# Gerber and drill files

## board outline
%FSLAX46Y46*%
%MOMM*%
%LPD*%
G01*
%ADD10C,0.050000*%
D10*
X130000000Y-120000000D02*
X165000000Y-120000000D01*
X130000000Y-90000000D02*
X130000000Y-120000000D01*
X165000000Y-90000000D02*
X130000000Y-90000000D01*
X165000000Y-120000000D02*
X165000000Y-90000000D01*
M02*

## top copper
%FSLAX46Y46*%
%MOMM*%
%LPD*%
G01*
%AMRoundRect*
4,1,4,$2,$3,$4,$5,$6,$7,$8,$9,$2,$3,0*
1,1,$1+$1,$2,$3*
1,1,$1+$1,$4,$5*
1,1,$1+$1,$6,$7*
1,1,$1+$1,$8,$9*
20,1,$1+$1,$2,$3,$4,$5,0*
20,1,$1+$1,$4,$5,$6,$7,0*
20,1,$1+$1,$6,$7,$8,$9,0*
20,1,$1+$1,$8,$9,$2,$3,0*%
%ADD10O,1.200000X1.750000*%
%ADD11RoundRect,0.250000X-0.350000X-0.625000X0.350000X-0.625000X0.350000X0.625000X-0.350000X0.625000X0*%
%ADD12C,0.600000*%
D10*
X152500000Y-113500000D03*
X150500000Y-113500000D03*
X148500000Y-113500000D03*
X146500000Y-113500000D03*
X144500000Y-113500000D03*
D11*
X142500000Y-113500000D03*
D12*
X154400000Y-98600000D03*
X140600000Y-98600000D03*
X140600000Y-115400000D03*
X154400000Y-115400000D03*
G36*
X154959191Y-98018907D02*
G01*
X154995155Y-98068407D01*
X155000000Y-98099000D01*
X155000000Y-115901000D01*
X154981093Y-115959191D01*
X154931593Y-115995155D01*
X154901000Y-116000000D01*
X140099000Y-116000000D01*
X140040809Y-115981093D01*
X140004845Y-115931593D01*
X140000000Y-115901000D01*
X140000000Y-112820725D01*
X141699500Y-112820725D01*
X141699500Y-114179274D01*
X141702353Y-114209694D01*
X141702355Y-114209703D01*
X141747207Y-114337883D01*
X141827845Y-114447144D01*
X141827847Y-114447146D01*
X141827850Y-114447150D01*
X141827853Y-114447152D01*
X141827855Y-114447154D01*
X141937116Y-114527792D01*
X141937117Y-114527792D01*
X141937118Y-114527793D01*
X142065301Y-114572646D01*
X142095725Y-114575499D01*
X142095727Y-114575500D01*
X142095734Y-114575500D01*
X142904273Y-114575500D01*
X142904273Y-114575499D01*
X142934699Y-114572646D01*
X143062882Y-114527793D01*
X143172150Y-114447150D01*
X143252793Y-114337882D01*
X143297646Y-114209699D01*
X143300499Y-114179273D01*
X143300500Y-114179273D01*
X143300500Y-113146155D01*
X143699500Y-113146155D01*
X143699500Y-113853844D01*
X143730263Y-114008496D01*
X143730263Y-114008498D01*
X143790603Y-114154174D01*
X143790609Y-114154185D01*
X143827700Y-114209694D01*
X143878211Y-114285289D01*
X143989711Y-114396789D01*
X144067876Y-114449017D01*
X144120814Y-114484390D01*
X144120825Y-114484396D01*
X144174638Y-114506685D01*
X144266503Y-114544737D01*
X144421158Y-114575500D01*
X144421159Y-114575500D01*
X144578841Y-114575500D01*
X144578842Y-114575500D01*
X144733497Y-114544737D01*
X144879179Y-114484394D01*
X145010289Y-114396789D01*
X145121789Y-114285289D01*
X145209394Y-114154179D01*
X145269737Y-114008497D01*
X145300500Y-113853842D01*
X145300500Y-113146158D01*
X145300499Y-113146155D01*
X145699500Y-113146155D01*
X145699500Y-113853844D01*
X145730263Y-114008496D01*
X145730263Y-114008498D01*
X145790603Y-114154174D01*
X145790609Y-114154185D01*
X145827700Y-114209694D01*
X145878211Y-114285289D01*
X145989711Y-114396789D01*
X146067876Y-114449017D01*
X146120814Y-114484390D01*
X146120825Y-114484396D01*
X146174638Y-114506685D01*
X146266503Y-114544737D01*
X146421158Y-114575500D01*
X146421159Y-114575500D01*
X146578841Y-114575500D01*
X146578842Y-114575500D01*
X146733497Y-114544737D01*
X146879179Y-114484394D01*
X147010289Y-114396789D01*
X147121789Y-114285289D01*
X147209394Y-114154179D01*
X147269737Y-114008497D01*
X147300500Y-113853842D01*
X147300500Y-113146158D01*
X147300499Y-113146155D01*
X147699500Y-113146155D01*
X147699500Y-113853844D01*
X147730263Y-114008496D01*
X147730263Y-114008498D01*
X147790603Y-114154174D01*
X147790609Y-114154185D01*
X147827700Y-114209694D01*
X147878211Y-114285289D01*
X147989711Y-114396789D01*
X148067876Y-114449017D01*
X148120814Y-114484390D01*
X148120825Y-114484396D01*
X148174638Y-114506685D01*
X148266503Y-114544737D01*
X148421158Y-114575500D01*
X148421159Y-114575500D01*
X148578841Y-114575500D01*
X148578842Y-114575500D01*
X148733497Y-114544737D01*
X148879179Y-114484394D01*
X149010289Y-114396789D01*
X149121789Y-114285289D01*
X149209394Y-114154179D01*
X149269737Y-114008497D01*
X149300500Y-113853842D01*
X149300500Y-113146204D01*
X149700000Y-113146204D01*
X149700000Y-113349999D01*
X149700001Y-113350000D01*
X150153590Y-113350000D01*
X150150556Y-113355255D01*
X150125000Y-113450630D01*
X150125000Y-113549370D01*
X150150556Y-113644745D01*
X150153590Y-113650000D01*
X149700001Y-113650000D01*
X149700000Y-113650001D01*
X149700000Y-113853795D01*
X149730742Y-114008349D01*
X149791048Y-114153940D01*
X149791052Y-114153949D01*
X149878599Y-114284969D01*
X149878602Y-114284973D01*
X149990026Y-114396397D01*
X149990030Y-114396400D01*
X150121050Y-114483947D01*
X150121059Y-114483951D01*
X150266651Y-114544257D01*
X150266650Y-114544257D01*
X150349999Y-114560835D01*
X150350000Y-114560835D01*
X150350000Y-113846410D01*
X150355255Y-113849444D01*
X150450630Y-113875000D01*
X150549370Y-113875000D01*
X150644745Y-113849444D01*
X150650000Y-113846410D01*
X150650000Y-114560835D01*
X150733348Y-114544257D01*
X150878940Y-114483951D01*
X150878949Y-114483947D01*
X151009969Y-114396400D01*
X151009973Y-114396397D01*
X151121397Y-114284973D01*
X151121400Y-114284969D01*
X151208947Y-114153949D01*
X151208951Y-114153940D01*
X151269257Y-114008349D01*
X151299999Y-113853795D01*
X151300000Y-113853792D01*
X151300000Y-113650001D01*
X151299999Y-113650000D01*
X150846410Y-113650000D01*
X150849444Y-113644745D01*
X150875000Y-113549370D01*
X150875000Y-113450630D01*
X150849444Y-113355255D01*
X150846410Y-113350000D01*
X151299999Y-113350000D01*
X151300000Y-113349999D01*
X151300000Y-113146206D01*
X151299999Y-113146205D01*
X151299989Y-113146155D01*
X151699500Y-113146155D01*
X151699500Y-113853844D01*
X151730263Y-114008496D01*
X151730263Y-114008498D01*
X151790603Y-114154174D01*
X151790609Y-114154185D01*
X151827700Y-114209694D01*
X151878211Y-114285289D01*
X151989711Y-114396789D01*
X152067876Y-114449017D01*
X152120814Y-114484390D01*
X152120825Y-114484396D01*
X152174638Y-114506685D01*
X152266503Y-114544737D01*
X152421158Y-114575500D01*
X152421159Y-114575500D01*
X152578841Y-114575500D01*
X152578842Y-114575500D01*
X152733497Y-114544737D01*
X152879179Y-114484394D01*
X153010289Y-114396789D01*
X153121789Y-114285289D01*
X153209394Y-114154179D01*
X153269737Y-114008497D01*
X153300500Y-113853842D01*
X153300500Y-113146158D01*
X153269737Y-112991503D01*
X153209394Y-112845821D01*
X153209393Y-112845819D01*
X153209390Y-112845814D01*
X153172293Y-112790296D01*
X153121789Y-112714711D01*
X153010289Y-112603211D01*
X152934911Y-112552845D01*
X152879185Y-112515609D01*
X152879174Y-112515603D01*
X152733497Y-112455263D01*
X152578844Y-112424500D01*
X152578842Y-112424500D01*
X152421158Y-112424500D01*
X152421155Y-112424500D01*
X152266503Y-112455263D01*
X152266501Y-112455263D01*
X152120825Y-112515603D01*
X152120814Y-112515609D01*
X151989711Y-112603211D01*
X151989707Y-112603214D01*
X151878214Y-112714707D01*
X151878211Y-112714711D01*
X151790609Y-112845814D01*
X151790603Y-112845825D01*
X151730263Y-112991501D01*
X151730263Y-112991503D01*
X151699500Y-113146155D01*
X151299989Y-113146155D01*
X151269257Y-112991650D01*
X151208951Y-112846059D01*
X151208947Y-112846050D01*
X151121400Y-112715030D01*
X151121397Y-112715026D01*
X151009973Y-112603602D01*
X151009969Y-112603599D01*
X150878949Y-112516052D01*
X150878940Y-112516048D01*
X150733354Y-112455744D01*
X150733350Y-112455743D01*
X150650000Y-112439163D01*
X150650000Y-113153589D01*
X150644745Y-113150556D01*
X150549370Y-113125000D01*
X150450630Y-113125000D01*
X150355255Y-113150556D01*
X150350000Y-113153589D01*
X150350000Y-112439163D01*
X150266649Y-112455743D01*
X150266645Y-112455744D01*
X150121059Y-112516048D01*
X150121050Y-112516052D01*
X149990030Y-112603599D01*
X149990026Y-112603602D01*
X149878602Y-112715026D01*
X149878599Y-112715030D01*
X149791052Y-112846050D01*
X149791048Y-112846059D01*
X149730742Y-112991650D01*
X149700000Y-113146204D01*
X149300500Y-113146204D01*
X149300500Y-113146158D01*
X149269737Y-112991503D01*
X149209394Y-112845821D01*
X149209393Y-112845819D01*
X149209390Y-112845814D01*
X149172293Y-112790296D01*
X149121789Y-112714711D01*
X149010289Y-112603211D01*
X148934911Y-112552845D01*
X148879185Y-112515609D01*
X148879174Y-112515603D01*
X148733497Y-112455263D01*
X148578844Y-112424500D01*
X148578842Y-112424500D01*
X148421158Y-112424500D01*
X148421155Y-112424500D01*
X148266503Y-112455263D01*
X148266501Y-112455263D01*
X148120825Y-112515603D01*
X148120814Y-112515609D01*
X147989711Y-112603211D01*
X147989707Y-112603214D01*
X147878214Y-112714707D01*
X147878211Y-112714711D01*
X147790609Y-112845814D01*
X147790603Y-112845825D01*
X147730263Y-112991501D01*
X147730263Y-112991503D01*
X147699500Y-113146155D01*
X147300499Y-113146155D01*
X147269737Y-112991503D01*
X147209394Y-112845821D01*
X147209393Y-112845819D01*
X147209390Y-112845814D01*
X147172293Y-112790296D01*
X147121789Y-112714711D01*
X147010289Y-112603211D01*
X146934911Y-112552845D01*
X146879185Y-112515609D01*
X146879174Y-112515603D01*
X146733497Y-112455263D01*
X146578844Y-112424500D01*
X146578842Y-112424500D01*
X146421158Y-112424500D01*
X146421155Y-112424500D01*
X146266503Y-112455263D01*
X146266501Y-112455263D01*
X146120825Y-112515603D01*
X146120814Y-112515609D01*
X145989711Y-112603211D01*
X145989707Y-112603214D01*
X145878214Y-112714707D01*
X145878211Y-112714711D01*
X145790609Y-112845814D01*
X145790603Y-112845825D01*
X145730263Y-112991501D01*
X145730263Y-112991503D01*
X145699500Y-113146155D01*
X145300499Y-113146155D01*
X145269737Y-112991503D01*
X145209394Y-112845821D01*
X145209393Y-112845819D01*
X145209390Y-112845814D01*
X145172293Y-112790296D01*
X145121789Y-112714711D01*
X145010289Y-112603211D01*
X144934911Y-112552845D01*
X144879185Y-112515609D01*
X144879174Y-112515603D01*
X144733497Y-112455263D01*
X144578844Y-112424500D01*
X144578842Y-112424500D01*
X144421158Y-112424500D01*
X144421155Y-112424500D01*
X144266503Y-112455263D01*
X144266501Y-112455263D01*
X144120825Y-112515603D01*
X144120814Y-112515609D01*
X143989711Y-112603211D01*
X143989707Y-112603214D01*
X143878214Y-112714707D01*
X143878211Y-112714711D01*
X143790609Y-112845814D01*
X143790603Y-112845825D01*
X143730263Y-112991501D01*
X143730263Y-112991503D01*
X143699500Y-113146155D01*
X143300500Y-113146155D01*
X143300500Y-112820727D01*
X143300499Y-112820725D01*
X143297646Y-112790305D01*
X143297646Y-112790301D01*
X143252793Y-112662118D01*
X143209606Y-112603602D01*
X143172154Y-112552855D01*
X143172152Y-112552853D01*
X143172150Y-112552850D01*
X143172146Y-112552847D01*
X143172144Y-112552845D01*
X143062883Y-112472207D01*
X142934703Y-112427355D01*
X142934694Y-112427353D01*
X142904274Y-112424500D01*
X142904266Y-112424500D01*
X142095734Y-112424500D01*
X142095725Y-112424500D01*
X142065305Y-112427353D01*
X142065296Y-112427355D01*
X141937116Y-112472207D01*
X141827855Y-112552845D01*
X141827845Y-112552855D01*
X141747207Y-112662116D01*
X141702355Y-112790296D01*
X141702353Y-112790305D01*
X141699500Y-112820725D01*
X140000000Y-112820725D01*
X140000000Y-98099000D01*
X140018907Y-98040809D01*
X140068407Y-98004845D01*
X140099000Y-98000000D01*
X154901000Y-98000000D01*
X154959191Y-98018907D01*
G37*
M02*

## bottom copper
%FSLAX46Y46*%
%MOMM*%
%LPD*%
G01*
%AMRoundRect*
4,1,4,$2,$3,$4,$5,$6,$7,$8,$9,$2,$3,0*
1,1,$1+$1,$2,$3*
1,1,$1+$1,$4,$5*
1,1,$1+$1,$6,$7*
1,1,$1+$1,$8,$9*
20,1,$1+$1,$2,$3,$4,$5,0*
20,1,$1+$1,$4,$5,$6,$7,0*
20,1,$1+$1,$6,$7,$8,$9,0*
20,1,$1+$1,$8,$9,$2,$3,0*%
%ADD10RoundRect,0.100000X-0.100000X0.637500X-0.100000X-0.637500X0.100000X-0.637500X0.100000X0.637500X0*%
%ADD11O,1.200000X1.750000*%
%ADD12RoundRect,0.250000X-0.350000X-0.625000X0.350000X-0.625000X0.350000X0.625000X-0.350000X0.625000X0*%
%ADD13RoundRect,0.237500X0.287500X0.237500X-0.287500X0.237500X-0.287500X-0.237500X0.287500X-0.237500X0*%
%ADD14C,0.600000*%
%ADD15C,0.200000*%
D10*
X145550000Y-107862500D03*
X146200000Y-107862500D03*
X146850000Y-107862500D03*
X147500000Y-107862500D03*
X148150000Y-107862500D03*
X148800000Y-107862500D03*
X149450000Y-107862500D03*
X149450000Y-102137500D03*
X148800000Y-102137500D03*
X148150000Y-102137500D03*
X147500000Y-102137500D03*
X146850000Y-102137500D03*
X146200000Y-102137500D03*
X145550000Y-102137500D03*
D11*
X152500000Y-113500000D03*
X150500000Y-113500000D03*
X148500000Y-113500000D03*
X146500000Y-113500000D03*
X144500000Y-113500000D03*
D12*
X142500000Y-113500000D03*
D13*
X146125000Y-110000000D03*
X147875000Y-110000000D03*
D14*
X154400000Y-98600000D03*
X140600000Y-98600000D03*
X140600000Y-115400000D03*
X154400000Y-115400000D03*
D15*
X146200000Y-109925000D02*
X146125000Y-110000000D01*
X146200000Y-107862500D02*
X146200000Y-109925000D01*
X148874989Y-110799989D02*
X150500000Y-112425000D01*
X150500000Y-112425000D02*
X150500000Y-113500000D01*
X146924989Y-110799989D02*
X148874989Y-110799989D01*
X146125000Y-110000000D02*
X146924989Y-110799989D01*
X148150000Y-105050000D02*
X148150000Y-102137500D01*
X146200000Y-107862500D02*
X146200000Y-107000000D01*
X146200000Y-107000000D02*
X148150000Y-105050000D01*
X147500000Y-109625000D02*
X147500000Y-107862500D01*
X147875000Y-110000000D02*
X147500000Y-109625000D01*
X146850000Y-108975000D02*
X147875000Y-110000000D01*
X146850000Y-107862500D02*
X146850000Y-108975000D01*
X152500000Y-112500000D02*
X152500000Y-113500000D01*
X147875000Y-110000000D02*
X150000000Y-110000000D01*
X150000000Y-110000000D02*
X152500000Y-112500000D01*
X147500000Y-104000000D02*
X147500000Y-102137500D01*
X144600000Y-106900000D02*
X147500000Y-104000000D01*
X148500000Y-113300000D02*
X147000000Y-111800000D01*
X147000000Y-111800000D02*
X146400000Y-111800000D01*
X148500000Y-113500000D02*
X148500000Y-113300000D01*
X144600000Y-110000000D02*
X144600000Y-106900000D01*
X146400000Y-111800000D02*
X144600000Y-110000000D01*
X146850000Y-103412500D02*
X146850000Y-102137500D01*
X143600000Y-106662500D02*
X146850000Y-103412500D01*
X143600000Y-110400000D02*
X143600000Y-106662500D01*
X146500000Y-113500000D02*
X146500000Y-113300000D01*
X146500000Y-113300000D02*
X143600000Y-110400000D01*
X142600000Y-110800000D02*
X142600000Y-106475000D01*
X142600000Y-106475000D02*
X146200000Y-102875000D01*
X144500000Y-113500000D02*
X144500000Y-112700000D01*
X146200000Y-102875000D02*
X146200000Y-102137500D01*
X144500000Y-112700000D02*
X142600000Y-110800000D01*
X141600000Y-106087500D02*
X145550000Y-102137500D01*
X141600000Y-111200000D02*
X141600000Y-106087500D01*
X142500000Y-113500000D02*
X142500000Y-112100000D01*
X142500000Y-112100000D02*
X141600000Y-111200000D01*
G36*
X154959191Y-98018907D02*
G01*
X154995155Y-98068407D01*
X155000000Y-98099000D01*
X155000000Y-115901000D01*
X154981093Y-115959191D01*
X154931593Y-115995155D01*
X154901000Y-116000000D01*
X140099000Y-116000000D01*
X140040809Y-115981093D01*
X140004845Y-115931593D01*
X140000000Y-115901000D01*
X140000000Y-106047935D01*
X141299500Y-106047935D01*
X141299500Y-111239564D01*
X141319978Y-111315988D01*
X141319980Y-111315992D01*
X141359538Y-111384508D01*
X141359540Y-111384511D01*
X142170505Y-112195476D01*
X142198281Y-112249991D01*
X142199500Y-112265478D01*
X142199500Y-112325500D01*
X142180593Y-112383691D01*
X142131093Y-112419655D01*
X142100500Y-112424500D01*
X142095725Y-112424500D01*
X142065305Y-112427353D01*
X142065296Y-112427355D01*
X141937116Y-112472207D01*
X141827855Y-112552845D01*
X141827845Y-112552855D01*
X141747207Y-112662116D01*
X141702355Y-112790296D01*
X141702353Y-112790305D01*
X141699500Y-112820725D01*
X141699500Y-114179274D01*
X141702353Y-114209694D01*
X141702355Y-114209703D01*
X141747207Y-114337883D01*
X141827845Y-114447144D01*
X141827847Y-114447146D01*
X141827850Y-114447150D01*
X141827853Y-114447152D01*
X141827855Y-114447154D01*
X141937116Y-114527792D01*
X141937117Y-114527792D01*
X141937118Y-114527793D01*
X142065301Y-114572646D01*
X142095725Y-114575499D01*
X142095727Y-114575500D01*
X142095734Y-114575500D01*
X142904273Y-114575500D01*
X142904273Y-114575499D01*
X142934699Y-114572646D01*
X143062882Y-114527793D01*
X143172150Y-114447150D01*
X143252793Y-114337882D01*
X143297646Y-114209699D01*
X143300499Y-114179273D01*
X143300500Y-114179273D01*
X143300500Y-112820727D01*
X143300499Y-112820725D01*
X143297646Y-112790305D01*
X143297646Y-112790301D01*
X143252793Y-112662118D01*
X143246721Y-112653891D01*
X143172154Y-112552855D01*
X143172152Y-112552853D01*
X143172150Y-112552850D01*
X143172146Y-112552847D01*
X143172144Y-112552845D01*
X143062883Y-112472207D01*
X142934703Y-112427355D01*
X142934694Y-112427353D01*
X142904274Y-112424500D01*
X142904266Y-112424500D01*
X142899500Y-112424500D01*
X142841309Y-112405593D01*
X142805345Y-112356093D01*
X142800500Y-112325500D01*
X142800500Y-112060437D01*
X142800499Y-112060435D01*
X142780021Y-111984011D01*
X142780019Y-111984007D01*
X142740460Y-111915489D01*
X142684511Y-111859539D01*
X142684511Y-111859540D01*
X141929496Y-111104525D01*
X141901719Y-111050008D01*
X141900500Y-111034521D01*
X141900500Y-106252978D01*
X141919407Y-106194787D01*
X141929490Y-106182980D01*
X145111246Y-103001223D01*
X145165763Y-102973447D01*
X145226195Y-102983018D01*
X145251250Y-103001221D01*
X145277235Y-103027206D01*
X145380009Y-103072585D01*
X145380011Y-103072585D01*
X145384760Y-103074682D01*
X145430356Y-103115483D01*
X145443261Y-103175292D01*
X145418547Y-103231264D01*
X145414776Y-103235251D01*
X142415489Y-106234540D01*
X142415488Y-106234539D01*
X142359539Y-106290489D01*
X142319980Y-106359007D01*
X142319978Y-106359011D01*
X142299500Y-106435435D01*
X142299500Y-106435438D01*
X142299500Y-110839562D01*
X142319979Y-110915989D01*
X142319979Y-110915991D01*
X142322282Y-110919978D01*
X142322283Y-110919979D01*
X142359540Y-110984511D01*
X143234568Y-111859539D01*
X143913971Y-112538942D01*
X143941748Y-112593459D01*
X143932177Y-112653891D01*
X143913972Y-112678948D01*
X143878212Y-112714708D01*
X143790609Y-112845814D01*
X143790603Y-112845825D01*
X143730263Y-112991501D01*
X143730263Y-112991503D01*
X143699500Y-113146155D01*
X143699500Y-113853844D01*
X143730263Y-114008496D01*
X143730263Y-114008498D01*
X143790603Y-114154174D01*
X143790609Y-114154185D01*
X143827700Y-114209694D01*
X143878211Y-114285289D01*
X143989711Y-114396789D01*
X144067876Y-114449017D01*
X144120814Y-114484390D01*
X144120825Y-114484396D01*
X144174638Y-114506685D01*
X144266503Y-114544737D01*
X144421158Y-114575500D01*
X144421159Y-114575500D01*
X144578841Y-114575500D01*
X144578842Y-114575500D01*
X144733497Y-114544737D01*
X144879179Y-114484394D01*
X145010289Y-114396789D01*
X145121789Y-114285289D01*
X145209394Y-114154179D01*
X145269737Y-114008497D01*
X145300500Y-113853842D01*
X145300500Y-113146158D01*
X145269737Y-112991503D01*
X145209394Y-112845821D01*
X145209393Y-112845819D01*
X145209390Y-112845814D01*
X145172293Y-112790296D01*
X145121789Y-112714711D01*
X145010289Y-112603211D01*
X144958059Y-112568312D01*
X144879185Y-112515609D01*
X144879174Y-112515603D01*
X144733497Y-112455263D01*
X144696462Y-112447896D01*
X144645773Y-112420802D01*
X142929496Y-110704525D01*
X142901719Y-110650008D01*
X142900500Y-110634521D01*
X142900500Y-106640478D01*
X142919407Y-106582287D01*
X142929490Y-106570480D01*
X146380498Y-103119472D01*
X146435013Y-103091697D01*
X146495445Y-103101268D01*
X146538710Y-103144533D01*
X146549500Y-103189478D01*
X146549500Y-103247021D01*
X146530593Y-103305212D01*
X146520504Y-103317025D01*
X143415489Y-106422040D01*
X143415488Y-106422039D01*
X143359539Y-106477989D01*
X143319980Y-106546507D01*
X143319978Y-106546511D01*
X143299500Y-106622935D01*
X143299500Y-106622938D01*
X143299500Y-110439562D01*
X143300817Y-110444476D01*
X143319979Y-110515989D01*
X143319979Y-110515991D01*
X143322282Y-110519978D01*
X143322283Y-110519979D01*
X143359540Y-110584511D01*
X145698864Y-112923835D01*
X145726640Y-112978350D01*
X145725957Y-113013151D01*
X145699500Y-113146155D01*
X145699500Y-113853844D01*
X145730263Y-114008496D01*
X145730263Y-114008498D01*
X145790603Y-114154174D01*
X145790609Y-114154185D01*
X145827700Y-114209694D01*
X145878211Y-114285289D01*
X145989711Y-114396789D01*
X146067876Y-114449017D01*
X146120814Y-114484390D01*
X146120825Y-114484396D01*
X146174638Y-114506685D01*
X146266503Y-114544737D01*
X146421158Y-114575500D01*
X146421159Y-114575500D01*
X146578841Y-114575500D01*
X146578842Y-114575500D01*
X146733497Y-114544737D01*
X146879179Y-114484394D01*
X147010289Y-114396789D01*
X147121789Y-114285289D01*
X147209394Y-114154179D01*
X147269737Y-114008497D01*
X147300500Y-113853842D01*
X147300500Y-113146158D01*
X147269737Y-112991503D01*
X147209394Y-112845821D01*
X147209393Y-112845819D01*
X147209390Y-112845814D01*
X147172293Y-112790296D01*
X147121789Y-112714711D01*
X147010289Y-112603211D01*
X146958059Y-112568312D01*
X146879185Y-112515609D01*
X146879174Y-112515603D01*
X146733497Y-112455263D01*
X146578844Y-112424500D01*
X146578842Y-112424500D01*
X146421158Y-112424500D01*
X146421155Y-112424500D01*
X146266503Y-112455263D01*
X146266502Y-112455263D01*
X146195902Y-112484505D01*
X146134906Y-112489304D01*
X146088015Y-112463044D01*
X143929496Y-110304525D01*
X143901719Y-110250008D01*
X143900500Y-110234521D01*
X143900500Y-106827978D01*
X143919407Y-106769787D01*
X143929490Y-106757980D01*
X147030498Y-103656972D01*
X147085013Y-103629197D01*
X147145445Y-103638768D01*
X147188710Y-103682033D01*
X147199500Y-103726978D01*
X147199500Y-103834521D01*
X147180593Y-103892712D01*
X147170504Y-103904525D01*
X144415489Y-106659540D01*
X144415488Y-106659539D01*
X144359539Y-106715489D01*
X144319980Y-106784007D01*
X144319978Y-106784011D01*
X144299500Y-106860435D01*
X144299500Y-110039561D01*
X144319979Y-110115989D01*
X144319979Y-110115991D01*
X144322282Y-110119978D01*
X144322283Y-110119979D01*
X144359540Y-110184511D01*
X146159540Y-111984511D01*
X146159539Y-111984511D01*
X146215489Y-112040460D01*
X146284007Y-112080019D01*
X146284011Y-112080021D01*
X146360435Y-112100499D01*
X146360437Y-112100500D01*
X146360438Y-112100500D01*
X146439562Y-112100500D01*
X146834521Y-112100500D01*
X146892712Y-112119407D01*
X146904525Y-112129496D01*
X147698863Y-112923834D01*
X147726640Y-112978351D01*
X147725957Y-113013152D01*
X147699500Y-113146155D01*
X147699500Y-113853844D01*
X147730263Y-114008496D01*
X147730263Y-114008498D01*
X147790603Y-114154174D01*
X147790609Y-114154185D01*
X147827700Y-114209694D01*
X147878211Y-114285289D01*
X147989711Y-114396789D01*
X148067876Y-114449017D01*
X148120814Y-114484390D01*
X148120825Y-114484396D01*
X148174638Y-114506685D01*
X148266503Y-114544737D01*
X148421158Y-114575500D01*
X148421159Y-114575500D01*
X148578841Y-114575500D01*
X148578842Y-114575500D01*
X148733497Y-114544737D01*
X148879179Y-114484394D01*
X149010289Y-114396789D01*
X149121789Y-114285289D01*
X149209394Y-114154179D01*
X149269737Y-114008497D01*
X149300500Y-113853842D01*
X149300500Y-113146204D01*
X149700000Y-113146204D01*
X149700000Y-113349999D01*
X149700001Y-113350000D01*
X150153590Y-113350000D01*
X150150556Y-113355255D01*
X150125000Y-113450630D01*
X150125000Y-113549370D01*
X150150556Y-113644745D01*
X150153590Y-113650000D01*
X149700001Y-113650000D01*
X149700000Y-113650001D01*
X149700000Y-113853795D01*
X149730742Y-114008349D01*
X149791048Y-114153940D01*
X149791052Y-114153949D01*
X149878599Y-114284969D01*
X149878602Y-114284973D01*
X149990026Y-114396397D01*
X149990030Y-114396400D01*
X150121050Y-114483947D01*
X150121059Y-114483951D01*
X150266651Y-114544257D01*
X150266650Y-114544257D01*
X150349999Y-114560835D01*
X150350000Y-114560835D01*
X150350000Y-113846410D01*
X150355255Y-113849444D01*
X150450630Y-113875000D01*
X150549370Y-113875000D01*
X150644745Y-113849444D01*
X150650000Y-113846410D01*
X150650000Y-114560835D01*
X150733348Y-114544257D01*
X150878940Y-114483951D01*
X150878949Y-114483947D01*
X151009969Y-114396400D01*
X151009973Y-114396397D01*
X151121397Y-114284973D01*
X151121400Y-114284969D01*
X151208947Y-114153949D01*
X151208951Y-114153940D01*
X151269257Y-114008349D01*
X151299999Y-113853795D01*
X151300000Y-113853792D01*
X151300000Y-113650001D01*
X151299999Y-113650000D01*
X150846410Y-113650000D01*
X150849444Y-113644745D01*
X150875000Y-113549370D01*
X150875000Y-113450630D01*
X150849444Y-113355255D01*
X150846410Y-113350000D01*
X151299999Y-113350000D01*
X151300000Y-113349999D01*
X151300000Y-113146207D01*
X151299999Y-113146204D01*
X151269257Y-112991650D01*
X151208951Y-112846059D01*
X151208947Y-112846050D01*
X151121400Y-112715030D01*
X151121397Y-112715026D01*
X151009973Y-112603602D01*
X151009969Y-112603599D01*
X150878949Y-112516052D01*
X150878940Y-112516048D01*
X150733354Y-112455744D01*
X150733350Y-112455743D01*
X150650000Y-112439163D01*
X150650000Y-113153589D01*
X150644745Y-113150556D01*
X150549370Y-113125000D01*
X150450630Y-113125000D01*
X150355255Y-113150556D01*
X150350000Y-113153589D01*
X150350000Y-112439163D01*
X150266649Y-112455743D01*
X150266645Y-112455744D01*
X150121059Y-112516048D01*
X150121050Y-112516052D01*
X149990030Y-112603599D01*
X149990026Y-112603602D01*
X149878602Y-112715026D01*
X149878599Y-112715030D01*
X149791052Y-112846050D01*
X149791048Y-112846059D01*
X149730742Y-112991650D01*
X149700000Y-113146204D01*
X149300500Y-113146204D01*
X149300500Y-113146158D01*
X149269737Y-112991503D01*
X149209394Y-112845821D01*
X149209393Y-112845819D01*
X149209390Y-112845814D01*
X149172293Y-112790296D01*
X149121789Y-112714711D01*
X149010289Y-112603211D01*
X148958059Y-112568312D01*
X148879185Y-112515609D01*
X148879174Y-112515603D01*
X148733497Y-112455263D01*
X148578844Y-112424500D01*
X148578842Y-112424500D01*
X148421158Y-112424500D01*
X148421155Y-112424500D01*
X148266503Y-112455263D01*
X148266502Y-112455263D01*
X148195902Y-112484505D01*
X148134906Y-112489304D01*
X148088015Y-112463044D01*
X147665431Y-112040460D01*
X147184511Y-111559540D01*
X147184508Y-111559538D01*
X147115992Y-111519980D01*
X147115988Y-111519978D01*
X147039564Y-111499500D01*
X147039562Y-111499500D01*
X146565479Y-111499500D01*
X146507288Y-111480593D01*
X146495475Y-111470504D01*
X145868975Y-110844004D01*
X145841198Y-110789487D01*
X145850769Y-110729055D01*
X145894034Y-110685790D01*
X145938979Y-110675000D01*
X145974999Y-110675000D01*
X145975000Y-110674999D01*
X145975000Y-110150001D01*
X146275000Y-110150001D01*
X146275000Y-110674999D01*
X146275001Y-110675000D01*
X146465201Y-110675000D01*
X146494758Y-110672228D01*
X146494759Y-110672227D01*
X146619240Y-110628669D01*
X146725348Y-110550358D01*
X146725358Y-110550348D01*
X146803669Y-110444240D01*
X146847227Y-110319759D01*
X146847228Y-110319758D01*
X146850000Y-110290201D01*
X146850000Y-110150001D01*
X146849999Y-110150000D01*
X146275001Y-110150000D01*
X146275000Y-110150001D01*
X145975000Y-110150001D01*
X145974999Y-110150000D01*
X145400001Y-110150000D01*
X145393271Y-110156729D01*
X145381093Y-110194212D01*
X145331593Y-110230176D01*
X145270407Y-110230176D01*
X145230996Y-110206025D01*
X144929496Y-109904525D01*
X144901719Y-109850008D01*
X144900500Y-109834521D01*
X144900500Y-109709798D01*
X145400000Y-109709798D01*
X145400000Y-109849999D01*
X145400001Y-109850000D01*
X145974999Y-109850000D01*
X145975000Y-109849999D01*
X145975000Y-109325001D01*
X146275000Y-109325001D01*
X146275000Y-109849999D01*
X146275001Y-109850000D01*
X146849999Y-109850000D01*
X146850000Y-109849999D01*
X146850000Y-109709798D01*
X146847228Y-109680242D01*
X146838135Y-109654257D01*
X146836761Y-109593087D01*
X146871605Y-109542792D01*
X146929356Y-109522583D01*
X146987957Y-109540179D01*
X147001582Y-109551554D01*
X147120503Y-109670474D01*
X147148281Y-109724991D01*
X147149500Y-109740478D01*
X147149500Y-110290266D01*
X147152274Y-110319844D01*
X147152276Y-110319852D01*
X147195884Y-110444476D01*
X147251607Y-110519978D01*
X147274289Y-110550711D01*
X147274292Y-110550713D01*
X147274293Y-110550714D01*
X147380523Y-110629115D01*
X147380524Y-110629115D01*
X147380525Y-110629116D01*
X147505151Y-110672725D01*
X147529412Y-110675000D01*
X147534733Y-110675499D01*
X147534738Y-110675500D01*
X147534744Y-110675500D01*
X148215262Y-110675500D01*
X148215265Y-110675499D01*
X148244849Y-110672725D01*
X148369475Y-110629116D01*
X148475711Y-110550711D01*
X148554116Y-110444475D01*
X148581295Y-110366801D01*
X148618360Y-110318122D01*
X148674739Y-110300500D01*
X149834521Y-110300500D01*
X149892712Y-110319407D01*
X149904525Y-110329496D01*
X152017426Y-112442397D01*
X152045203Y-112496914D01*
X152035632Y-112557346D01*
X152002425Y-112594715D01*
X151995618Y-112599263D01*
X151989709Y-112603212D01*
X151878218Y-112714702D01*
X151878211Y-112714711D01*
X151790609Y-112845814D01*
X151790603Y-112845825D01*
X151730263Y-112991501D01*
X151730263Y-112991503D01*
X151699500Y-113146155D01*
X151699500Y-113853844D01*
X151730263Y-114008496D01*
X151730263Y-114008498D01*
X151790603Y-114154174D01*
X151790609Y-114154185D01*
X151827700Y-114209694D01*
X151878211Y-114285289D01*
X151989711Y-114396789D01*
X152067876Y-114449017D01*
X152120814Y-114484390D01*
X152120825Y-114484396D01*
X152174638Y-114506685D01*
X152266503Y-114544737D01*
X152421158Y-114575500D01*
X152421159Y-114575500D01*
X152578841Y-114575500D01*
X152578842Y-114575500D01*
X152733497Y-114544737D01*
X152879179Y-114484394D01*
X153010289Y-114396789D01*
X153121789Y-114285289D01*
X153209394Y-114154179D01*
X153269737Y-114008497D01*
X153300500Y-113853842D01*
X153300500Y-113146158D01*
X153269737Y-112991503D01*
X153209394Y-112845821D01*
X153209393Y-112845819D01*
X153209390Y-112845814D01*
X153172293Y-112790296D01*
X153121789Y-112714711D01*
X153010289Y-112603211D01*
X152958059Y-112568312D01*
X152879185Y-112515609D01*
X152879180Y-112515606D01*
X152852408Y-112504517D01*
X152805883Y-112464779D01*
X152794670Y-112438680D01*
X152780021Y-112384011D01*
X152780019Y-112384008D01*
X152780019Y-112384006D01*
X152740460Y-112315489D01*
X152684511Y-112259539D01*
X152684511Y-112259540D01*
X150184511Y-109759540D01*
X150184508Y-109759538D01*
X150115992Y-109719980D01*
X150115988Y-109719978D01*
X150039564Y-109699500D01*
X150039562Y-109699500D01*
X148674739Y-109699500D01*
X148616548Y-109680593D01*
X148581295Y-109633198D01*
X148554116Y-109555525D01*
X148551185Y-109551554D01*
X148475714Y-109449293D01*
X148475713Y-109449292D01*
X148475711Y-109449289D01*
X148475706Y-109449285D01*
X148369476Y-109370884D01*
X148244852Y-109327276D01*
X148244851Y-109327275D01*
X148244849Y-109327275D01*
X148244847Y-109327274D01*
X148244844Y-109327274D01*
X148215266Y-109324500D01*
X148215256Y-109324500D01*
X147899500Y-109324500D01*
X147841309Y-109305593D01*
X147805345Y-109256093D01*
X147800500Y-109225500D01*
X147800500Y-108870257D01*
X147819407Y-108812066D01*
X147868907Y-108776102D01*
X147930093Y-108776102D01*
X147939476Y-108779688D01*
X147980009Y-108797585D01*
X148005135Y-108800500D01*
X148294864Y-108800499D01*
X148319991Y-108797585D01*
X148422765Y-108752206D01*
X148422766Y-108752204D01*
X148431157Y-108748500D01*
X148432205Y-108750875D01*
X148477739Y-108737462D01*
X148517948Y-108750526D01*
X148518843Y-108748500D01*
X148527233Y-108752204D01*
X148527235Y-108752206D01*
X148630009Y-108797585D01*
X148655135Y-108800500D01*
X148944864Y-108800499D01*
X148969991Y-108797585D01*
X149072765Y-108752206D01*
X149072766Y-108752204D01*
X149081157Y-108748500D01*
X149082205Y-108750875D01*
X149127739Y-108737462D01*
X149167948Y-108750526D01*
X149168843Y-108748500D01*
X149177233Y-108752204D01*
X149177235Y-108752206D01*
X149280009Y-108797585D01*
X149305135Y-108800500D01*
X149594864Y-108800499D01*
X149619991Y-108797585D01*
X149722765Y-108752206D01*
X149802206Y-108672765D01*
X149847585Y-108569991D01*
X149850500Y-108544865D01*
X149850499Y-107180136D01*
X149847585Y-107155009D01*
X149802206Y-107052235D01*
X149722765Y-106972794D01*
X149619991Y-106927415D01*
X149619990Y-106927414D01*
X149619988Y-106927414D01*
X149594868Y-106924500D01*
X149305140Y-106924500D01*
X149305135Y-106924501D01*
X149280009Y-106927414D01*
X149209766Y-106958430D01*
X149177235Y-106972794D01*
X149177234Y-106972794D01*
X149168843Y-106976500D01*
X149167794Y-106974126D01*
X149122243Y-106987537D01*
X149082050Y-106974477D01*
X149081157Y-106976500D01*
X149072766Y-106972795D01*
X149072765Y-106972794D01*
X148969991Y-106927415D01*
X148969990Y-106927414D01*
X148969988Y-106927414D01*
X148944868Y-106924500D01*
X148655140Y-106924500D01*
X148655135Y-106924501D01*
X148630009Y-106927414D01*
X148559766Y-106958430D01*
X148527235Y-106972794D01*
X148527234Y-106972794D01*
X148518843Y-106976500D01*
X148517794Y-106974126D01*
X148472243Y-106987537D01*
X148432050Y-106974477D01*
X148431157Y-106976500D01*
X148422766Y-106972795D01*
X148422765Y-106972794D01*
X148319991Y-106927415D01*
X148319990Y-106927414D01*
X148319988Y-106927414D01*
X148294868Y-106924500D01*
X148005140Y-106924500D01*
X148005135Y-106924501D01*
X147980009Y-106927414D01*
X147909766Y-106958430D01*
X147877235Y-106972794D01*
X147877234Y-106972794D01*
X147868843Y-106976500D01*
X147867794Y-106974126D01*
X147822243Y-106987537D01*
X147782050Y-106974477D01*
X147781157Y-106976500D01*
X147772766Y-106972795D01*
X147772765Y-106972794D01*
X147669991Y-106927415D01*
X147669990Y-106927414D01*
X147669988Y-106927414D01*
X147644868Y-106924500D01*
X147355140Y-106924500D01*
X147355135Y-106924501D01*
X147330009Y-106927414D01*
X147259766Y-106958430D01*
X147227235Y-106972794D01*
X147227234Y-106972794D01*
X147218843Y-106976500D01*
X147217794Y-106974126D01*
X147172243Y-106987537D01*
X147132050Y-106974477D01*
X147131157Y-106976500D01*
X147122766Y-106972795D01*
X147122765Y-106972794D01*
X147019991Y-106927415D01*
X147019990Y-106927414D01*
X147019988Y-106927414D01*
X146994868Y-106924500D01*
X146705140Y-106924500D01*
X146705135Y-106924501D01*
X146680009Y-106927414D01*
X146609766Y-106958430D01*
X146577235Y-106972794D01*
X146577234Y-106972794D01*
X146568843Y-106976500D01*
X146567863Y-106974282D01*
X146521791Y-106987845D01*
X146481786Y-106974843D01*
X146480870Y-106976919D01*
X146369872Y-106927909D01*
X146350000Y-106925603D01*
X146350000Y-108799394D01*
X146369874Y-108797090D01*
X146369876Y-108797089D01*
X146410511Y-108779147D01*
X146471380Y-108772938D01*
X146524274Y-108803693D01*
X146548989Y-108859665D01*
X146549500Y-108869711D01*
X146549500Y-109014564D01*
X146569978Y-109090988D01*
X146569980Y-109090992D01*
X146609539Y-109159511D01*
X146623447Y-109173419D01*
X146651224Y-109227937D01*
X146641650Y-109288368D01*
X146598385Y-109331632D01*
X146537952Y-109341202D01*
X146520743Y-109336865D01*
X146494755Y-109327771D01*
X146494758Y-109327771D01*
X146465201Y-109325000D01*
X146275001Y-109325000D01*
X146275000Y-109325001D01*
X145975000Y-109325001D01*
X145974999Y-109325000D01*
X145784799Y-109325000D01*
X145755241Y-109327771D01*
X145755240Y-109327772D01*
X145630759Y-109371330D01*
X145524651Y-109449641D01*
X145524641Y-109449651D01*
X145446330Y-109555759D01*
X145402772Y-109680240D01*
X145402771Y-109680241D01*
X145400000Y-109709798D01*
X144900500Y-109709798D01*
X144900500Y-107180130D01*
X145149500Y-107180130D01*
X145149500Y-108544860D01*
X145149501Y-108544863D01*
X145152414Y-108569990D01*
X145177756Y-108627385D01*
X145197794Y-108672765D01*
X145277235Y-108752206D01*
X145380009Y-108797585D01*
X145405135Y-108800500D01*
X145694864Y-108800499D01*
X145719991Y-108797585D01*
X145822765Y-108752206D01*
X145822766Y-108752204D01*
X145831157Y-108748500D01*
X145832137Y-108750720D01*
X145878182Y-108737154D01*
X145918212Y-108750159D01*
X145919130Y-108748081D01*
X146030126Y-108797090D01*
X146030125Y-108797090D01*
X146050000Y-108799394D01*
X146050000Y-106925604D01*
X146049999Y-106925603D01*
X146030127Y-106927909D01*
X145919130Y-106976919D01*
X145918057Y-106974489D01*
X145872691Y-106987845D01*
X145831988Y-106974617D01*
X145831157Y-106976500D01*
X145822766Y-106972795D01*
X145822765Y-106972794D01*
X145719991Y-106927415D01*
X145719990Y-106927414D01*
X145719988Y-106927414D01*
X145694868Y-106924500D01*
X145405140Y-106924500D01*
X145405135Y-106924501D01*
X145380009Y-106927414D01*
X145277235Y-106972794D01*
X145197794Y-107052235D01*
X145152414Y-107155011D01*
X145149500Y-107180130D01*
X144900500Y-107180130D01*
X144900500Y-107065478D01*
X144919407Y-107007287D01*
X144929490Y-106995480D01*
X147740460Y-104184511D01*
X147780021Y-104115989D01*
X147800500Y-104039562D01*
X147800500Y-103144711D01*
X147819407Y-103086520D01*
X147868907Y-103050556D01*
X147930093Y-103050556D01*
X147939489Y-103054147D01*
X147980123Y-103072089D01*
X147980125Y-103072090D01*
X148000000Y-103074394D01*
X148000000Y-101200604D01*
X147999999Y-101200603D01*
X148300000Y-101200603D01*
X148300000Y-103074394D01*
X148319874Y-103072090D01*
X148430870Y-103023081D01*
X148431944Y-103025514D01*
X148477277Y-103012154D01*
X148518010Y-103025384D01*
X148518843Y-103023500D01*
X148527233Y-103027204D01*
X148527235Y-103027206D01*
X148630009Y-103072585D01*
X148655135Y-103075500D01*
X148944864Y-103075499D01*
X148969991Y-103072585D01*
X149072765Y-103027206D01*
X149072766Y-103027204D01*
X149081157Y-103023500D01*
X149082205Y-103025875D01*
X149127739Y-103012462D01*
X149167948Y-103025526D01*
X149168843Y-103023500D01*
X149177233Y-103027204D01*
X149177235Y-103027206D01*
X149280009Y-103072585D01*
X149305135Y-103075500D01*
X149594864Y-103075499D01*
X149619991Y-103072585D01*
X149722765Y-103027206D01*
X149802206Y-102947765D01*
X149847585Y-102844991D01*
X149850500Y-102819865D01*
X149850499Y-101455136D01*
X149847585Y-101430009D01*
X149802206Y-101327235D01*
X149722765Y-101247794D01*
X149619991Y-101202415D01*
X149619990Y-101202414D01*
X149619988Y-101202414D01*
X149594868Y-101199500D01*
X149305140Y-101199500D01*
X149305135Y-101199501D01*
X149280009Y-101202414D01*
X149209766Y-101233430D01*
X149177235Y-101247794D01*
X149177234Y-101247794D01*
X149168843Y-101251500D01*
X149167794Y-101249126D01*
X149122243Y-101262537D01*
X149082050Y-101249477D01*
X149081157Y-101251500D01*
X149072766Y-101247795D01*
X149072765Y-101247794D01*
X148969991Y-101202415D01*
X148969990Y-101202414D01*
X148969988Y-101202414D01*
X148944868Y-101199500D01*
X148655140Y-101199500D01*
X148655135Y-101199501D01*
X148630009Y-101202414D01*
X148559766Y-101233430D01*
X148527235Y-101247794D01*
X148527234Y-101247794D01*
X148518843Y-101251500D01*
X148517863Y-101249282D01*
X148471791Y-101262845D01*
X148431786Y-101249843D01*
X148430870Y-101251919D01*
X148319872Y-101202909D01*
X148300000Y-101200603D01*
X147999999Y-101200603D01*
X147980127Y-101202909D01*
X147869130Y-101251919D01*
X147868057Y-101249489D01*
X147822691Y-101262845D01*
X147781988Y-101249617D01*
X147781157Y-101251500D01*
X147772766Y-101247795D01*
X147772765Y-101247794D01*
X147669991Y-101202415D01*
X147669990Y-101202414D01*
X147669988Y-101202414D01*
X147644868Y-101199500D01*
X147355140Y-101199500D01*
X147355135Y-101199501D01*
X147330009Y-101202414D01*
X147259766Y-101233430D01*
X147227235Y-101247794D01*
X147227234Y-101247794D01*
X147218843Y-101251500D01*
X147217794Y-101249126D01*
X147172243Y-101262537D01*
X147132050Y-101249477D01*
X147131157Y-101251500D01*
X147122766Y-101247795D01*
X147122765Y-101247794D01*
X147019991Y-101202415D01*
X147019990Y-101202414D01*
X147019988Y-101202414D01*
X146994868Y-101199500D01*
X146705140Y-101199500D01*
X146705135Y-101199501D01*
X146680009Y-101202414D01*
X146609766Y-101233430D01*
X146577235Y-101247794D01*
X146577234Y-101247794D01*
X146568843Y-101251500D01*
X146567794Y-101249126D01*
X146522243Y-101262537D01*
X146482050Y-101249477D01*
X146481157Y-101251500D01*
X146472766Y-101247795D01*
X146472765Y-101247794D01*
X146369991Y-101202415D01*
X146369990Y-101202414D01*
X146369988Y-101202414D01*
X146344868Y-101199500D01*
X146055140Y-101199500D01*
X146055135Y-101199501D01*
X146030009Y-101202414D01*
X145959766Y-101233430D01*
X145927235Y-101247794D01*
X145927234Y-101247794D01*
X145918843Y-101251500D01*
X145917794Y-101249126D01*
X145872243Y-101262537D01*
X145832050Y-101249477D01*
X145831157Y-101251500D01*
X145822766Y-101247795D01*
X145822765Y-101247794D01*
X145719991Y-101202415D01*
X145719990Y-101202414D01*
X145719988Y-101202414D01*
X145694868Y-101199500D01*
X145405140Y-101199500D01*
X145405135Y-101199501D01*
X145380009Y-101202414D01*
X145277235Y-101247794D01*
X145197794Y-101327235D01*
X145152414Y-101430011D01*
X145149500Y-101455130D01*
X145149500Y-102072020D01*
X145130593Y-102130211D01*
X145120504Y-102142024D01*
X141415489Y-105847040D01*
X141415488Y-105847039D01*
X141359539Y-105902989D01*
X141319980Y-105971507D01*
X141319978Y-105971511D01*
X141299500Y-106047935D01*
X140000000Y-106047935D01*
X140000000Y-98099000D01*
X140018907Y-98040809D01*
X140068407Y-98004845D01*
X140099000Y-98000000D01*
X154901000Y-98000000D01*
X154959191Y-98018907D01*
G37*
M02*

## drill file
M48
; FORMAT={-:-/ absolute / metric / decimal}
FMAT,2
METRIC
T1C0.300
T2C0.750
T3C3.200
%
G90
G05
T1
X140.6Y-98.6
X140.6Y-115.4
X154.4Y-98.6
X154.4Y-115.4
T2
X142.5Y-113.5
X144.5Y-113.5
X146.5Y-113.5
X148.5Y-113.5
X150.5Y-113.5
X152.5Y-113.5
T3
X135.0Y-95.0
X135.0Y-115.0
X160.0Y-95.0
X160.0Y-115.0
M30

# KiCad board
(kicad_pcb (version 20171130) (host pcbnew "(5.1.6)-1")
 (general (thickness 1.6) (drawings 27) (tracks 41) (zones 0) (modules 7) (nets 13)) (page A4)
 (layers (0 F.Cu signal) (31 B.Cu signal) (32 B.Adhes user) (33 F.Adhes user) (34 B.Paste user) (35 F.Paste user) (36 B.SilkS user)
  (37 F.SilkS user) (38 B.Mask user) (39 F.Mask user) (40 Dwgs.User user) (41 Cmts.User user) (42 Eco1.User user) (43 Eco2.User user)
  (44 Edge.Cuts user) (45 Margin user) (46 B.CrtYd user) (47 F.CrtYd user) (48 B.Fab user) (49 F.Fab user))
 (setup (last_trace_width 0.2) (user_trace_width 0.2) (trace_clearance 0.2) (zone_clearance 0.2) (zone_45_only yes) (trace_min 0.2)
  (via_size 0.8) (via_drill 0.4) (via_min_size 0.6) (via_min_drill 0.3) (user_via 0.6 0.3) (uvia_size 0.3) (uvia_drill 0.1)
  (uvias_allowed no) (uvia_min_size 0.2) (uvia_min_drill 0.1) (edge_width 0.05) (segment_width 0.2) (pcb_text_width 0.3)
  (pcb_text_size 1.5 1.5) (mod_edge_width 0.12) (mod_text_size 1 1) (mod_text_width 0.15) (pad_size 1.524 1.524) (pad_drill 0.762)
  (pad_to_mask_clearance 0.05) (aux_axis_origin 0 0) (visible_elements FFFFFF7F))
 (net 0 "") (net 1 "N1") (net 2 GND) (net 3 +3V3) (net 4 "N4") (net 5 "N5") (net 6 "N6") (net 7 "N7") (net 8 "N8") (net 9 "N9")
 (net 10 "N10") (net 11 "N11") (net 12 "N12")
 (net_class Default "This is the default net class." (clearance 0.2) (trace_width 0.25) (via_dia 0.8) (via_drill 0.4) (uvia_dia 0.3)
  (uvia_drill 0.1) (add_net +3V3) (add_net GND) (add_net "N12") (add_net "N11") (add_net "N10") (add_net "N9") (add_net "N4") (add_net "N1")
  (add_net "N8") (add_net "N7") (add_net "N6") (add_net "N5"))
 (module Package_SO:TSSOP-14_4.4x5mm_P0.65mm (layer B.Cu) (at 147.5 105 270)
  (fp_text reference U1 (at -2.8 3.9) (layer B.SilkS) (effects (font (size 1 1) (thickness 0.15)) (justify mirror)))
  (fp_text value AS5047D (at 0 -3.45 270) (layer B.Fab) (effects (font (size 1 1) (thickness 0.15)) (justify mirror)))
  (pad 14 smd roundrect (at 2.8625 1.95 270) (size 1.475 0.4) (layers B.Cu B.Paste B.Mask) (roundrect_rratio 0.25) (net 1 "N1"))
  (pad 13 smd roundrect (at 2.8625 1.3 270) (size 1.475 0.4) (layers B.Cu B.Paste B.Mask) (roundrect_rratio 0.25) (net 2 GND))
  (pad 12 smd roundrect (at 2.8625 0.65 270) (size 1.475 0.4) (layers B.Cu B.Paste B.Mask) (roundrect_rratio 0.25) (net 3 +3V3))
  (pad 11 smd roundrect (at 2.8625 0 270) (size 1.475 0.4) (layers B.Cu B.Paste B.Mask) (roundrect_rratio 0.25) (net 3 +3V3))
  (pad 10 smd roundrect (at 2.8625 -0.65 270) (size 1.475 0.4) (layers B.Cu B.Paste B.Mask) (roundrect_rratio 0.25) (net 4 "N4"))
  (pad 9 smd roundrect (at 2.8625 -1.3 270) (size 1.475 0.4) (layers B.Cu B.Paste B.Mask) (roundrect_rratio 0.25) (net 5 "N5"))
  (pad 8 smd roundrect (at 2.8625 -1.95 270) (size 1.475 0.4) (layers B.Cu B.Paste B.Mask) (roundrect_rratio 0.25) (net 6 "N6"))
  (pad 7 smd roundrect (at -2.8625 -1.95 270) (size 1.475 0.4) (layers B.Cu B.Paste B.Mask) (roundrect_rratio 0.25) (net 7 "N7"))
  (pad 6 smd roundrect (at -2.8625 -1.3 270) (size 1.475 0.4) (layers B.Cu B.Paste B.Mask) (roundrect_rratio 0.25) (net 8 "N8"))
  (pad 5 smd roundrect (at -2.8625 -0.65 270) (size 1.475 0.4) (layers B.Cu B.Paste B.Mask) (roundrect_rratio 0.25) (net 2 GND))
  (pad 4 smd roundrect (at -2.8625 0 270) (size 1.475 0.4) (layers B.Cu B.Paste B.Mask) (roundrect_rratio 0.25) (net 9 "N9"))
  (pad 3 smd roundrect (at -2.8625 0.65 270) (size 1.475 0.4) (layers B.Cu B.Paste B.Mask) (roundrect_rratio 0.25) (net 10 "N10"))
  (pad 2 smd roundrect (at -2.8625 1.3 270) (size 1.475 0.4) (layers B.Cu B.Paste B.Mask) (roundrect_rratio 0.25) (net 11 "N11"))
  (pad 1 smd roundrect (at -2.8625 1.95 270) (size 1.475 0.4) (layers B.Cu B.Paste B.Mask) (roundrect_rratio 0.25) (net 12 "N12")))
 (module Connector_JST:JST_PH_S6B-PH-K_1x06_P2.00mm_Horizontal (layer F.Cu) (at 142.5 113.5)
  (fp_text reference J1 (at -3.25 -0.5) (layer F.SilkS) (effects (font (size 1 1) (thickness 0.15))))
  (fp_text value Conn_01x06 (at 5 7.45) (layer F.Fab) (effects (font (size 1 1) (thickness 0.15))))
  (pad 6 thru_hole oval (at 10 0) (size 1.2 1.75) (drill 0.75) (layers *.Cu *.Mask) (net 3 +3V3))
  (pad 5 thru_hole oval (at 8 0) (size 1.2 1.75) (drill 0.75) (layers *.Cu *.Mask) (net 2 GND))
  (pad 4 thru_hole oval (at 6 0) (size 1.2 1.75) (drill 0.75) (layers *.Cu *.Mask) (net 9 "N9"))
  (pad 3 thru_hole oval (at 4 0) (size 1.2 1.75) (drill 0.75) (layers *.Cu *.Mask) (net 10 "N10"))
  (pad 2 thru_hole oval (at 2 0) (size 1.2 1.75) (drill 0.75) (layers *.Cu *.Mask) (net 11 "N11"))
  (pad 1 thru_hole roundrect (at 0 0) (size 1.2 1.75) (drill 0.75) (layers *.Cu *.Mask) (roundrect_rratio 0.208333) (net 12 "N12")))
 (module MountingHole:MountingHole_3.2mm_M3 (layer F.Cu) (at 160 115)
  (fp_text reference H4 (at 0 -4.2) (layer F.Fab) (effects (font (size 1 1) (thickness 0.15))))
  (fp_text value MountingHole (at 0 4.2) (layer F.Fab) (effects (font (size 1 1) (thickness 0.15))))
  (pad 1 np_thru_hole circle (at 0 0) (size 3.2 3.2) (drill 3.2) (layers *.Cu *.Mask)))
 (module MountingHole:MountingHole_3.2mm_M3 (layer F.Cu) (at 135 115)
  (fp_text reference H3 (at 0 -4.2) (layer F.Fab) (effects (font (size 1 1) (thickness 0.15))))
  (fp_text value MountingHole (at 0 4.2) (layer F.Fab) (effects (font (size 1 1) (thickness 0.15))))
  (pad 1 np_thru_hole circle (at 0 0) (size 3.2 3.2) (drill 3.2) (layers *.Cu *.Mask)))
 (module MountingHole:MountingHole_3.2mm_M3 (layer F.Cu) (at 160 95)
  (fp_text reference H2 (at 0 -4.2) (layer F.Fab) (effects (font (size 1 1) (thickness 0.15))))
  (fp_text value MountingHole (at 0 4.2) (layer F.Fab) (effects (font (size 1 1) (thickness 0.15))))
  (pad 1 np_thru_hole circle (at 0 0) (size 3.2 3.2) (drill 3.2) (layers *.Cu *.Mask)))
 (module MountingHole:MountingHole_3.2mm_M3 (layer F.Cu) (at 135 95)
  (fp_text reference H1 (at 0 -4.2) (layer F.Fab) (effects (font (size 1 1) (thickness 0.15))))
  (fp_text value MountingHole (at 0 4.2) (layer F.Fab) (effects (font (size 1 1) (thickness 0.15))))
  (pad 1 np_thru_hole circle (at 0 0) (size 3.2 3.2) (drill 3.2) (layers *.Cu *.Mask)))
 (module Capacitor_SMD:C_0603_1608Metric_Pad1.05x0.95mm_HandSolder (layer B.Cu) (at 147 110 180)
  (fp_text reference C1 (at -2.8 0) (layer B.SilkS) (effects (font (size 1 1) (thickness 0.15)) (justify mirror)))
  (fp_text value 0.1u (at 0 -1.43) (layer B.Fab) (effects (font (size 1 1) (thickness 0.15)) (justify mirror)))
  (pad 2 smd roundrect (at 0.875 0 180) (size 1.05 0.95) (layers B.Cu B.Paste B.Mask) (roundrect_rratio 0.25) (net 2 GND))
  (pad 1 smd roundrect (at -0.875 0 180) (size 1.05 0.95) (layers B.Cu B.Paste B.Mask) (roundrect_rratio 0.25) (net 3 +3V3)))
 (gr_line (start 130 120) (end 165 120) (layer Edge.Cuts) (width 0.05))
 (gr_line (start 130 90) (end 130 120) (layer Edge.Cuts) (width 0.05))
 (gr_line (start 165 90) (end 130 90) (layer Edge.Cuts) (width 0.05))
 (gr_line (start 165 120) (end 165 90) (layer Edge.Cuts) (width 0.05))
 (segment (start 146.2 109.925) (end 146.125 110) (width 0.2) (layer B.Cu) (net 2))
 (segment (start 146.2 107.8625) (end 146.2 109.925) (width 0.2) (layer B.Cu) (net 2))
 (segment (start 148.874989 110.799989) (end 150.5 112.425) (width 0.2) (layer B.Cu) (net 2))
 (segment (start 150.5 112.425) (end 150.5 113.5) (width 0.2) (layer B.Cu) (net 2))
 (segment (start 146.924989 110.799989) (end 148.874989 110.799989) (width 0.2) (layer B.Cu) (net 2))
 (segment (start 146.125 110) (end 146.924989 110.799989) (width 0.2) (layer B.Cu) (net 2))
 (segment (start 148.15 105.05) (end 148.15 102.1375) (width 0.2) (layer B.Cu) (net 2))
 (segment (start 146.2 107.8625) (end 146.2 107) (width 0.2) (layer B.Cu) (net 2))
 (segment (start 146.2 107) (end 148.15 105.05) (width 0.2) (layer B.Cu) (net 2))
 (via (at 154.4 98.6) (size 0.6) (drill 0.3) (layers F.Cu B.Cu) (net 2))
 (via (at 140.6 98.6) (size 0.6) (drill 0.3) (layers F.Cu B.Cu) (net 2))
 (via (at 140.6 115.4) (size 0.6) (drill 0.3) (layers F.Cu B.Cu) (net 2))
 (via (at 154.4 115.4) (size 0.6) (drill 0.3) (layers F.Cu B.Cu) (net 2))
 (segment (start 147.5 109.625) (end 147.5 107.8625) (width 0.2) (layer B.Cu) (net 3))
 (segment (start 147.875 110) (end 147.5 109.625) (width 0.2) (layer B.Cu) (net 3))
 (segment (start 146.85 108.975) (end 147.875 110) (width 0.2) (layer B.Cu) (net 3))
 (segment (start 146.85 107.8625) (end 146.85 108.975) (width 0.2) (layer B.Cu) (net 3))
 (segment (start 152.5 112.5) (end 152.5 113.5) (width 0.2) (layer B.Cu) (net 3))
 (segment (start 147.875 110) (end 150 110) (width 0.2) (layer B.Cu) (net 3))
 (segment (start 150 110) (end 152.5 112.5) (width 0.2) (layer B.Cu) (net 3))
 (segment (start 147.5 104) (end 147.5 102.1375) (width 0.2) (layer B.Cu) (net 9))
 (segment (start 144.6 106.9) (end 147.5 104) (width 0.2) (layer B.Cu) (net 9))
 (segment (start 148.5 113.3) (end 147 111.8) (width 0.2) (layer B.Cu) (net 9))
 (segment (start 147 111.8) (end 146.4 111.8) (width 0.2) (layer B.Cu) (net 9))
 (segment (start 148.5 113.5) (end 148.5 113.3) (width 0.2) (layer B.Cu) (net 9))
 (segment (start 144.6 110) (end 144.6 106.9) (width 0.2) (layer B.Cu) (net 9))
 (segment (start 146.4 111.8) (end 144.6 110) (width 0.2) (layer B.Cu) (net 9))
 (segment (start 146.85 103.4125) (end 146.85 102.1375) (width 0.2) (layer B.Cu) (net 10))
 (segment (start 143.6 106.6625) (end 146.85 103.4125) (width 0.2) (layer B.Cu) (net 10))
 (segment (start 143.6 110.4) (end 143.6 106.6625) (width 0.2) (layer B.Cu) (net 10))
 (segment (start 146.5 113.5) (end 146.5 113.3) (width 0.2) (layer B.Cu) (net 10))
 (segment (start 146.5 113.3) (end 143.6 110.4) (width 0.2) (layer B.Cu) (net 10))
 (segment (start 142.6 110.8) (end 142.6 106.475) (width 0.2) (layer B.Cu) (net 11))
 (segment (start 142.6 106.475) (end 146.2 102.875) (width 0.2) (layer B.Cu) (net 11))
 (segment (start 144.5 113.5) (end 144.5 112.7) (width 0.2) (layer B.Cu) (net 11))
 (segment (start 146.2 102.875) (end 146.2 102.1375) (width 0.2) (layer B.Cu) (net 11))
 (segment (start 144.5 112.7) (end 142.6 110.8) (width 0.2) (layer B.Cu) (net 11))
 (segment (start 141.6 106.0875) (end 145.55 102.1375) (width 0.2) (layer B.Cu) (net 12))
 (segment (start 141.6 111.2) (end 141.6 106.0875) (width 0.2) (layer B.Cu) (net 12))
 (segment (start 142.5 113.5) (end 142.5 112.1) (width 0.2) (layer B.Cu) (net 12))
 (segment (start 142.5 112.1) (end 141.6 111.2) (width 0.2) (layer B.Cu) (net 12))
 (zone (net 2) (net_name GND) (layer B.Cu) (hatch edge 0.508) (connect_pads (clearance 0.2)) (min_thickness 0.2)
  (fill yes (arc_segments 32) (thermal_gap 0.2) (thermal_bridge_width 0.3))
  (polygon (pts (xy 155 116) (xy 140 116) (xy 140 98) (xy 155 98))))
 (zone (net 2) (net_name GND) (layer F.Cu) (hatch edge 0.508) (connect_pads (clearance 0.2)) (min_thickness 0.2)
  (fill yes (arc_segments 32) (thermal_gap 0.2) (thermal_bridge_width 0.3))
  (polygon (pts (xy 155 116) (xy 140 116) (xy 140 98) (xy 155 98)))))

